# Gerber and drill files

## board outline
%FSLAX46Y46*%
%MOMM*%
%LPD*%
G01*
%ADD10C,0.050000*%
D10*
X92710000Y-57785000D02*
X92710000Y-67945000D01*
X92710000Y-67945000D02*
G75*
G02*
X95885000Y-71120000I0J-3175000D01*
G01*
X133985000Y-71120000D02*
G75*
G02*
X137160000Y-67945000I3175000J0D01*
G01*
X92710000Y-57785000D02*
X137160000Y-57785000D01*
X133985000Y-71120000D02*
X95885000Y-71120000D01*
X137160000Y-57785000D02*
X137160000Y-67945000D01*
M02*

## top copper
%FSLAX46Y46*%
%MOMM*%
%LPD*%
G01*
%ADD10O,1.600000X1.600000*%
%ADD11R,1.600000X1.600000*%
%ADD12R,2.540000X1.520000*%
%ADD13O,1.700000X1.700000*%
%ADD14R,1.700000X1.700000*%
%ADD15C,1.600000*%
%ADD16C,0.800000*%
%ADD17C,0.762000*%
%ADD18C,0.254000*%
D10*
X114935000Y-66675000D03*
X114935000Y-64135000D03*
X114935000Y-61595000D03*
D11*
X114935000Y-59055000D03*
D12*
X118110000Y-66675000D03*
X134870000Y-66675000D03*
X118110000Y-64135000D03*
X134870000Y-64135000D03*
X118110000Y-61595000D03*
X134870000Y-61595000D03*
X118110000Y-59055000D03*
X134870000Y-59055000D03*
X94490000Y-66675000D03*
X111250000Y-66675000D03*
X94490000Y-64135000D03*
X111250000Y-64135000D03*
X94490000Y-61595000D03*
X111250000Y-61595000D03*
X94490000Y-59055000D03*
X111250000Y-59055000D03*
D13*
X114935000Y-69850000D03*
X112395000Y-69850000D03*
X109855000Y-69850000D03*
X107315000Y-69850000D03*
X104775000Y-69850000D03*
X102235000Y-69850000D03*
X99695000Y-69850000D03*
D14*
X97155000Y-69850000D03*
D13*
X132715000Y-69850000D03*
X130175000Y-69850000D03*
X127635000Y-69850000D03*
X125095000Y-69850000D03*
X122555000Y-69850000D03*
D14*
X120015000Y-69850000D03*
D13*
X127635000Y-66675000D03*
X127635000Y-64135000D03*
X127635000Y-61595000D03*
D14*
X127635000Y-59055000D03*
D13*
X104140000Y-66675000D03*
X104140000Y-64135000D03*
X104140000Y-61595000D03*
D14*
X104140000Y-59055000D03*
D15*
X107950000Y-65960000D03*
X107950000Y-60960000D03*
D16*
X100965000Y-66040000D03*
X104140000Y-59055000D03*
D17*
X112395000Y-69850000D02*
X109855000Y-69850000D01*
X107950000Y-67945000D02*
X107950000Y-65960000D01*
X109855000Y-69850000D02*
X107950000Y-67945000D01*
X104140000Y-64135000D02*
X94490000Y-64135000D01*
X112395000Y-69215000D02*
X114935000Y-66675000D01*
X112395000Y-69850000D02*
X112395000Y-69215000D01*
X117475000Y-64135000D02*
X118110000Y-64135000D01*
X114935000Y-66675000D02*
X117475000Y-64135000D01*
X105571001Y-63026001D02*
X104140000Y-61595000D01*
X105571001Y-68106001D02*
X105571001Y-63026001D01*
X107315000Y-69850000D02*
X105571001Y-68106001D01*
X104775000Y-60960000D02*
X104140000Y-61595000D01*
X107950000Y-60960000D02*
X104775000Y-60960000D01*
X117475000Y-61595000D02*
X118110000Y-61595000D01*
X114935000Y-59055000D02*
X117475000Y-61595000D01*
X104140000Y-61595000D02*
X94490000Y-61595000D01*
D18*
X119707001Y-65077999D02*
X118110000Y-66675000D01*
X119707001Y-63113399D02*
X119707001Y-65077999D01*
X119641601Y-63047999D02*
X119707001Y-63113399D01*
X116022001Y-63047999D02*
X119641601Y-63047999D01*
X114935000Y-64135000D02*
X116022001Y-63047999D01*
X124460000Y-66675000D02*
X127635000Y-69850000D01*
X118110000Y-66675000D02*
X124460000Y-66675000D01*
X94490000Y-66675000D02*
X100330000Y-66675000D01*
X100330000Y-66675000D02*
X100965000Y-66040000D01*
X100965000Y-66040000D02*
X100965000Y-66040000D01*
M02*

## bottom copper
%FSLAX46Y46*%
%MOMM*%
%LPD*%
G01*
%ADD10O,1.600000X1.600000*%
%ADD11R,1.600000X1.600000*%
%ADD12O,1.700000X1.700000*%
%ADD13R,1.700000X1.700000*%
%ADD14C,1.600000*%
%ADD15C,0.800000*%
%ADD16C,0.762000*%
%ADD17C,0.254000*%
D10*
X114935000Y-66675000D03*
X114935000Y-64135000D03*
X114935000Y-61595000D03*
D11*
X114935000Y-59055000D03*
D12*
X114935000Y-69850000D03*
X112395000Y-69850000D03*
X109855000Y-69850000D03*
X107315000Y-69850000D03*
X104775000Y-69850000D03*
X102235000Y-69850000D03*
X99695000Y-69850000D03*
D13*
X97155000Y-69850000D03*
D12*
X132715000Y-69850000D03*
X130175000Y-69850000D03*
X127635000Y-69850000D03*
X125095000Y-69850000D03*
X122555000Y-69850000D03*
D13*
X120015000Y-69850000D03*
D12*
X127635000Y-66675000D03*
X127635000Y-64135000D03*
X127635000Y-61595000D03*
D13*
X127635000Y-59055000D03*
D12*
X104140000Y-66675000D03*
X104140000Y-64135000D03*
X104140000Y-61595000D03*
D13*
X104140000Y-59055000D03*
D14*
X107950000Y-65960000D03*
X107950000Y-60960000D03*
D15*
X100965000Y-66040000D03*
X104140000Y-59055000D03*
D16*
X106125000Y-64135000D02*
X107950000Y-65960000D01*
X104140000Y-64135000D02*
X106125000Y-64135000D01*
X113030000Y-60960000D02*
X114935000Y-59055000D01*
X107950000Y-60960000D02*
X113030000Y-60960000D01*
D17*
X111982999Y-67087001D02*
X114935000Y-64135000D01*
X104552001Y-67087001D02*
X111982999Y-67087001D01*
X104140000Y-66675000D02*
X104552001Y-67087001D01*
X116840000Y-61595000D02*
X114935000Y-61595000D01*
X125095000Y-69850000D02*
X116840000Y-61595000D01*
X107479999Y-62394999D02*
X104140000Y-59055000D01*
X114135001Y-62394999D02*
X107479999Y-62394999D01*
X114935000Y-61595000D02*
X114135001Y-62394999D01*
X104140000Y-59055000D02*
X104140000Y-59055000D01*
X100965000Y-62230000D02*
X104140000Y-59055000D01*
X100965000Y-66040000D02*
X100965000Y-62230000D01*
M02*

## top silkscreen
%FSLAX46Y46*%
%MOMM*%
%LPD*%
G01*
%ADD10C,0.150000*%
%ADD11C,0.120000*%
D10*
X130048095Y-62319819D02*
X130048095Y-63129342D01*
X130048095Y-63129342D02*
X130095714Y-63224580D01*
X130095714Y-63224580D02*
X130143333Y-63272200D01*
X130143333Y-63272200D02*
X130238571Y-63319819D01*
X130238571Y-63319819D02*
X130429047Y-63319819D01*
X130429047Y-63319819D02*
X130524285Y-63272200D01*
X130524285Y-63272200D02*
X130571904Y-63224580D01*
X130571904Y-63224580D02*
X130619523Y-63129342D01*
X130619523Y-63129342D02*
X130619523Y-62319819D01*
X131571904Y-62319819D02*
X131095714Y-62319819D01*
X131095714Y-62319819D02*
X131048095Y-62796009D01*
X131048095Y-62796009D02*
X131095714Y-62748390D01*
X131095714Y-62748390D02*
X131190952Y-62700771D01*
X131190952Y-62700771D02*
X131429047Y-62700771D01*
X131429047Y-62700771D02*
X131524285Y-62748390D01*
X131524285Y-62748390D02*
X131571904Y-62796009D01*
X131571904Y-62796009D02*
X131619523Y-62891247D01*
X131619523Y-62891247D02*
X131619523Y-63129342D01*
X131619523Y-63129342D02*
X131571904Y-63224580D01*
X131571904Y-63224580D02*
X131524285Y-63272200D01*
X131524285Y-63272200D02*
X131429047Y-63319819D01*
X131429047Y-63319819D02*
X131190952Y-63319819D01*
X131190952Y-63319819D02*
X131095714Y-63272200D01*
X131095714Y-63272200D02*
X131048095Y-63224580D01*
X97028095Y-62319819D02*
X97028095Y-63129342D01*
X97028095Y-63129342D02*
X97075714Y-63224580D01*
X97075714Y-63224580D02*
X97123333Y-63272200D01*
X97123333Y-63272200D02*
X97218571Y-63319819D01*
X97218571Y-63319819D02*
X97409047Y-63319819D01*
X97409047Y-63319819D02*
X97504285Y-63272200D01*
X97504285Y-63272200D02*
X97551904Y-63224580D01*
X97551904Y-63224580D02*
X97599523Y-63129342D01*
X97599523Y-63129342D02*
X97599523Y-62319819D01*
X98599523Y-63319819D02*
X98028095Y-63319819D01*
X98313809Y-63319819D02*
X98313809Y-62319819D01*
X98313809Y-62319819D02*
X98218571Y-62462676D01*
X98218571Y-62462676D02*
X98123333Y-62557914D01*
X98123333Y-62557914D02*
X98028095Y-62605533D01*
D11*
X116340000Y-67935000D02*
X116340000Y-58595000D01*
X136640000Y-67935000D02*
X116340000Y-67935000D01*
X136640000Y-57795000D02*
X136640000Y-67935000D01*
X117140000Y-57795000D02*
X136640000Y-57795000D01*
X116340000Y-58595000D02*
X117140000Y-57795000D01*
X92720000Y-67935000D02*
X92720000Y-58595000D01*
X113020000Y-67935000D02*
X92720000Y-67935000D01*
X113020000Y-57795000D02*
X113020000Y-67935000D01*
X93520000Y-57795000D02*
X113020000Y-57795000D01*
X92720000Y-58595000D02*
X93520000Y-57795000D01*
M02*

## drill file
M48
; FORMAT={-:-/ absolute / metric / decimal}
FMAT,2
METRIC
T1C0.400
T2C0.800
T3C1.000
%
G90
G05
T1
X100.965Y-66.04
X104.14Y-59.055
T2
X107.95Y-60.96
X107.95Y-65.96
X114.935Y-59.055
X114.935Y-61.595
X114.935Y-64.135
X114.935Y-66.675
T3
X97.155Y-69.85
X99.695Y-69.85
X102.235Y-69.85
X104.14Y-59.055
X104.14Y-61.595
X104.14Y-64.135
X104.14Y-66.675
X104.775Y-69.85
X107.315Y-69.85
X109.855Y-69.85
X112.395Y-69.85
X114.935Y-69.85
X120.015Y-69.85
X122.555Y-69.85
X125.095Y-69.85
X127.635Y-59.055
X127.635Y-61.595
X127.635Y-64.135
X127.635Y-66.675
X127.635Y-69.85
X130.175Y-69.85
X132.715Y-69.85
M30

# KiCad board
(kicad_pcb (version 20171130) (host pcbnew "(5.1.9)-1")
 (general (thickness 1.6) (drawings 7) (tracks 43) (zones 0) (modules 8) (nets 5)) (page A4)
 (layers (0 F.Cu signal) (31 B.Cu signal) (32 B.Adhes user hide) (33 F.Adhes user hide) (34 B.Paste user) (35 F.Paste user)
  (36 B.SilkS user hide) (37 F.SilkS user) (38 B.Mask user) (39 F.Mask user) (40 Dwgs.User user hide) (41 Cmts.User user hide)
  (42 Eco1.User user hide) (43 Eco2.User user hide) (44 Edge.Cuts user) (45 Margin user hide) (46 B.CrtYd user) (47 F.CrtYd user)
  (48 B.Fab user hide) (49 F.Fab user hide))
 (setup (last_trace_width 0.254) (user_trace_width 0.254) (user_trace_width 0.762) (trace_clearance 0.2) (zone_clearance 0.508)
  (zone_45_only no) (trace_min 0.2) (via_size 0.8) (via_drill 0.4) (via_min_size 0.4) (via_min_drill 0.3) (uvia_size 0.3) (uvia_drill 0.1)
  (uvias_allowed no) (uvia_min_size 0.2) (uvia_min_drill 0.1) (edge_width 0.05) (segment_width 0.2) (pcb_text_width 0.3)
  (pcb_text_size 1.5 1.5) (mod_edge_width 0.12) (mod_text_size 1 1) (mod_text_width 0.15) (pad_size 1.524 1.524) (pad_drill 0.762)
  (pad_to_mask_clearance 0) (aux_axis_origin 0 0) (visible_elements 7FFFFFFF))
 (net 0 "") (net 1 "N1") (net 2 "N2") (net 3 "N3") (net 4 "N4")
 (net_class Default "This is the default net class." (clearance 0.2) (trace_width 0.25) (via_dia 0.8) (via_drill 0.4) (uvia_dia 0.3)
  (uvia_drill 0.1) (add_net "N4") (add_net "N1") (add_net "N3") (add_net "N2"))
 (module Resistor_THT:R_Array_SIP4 (layer B.Cu) (at 114.935 59.055 270)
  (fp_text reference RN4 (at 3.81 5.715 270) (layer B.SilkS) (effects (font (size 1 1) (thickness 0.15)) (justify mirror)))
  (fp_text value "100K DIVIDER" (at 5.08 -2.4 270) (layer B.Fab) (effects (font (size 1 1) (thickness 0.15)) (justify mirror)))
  (pad 4 thru_hole oval (at 7.62 0 270) (size 1.6 1.6) (drill 0.8) (layers *.Cu *.Mask) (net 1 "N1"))
  (pad 3 thru_hole oval (at 5.08 0 270) (size 1.6 1.6) (drill 0.8) (layers *.Cu *.Mask) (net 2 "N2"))
  (pad 2 thru_hole oval (at 2.54 0 270) (size 1.6 1.6) (drill 0.8) (layers *.Cu *.Mask) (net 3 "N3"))
  (pad 1 thru_hole rect (at 0 0 270) (size 1.6 1.6) (drill 0.8) (layers *.Cu *.Mask) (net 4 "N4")))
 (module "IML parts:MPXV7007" (layer F.Cu) (at 126.49 62.865 270)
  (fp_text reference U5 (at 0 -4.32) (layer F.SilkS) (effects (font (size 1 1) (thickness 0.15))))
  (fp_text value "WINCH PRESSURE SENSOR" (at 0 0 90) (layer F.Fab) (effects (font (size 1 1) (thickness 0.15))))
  (fp_line (start 5.07 10.15) (end -4.27 10.15) (layer F.SilkS) (width 0.12))
  (fp_line (start 5.07 -10.15) (end 5.07 10.15) (layer F.SilkS) (width 0.12))
  (fp_line (start -5.07 -10.15) (end 5.07 -10.15) (layer F.SilkS) (width 0.12))
  (fp_line (start -5.07 9.35) (end -5.07 -10.15) (layer F.SilkS) (width 0.12))
  (fp_line (start -4.27 10.15) (end -5.07 9.35) (layer F.SilkS) (width 0.12))
  (pad 4 smd rect (at 3.81 8.38 270) (size 1.52 2.54) (layers F.Cu F.Paste F.Mask) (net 2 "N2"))
  (pad 5 smd rect (at 3.81 -8.38 270) (size 1.52 2.54) (layers F.Cu F.Paste F.Mask))
  (pad 3 smd rect (at 1.27 8.38 270) (size 1.52 2.54) (layers F.Cu F.Paste F.Mask) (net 1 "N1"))
  (pad 6 smd rect (at 1.27 -8.38 270) (size 1.52 2.54) (layers F.Cu F.Paste F.Mask))
  (pad 2 smd rect (at -1.27 8.38 270) (size 1.52 2.54) (layers F.Cu F.Paste F.Mask) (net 4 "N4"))
  (pad 7 smd rect (at -1.27 -8.38 270) (size 1.52 2.54) (layers F.Cu F.Paste F.Mask))
  (pad 1 smd rect (at -3.81 8.38 270) (size 1.52 2.54) (layers F.Cu F.Paste F.Mask))
  (pad 8 smd rect (at -3.81 -8.38 270) (size 1.52 2.54) (layers F.Cu F.Paste F.Mask)))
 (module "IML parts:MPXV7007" (layer F.Cu) (at 102.87 62.865 270)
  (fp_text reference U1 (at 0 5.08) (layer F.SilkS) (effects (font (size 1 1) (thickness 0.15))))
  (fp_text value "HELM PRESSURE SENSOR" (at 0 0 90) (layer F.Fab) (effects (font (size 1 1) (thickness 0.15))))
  (fp_line (start 5.07 10.15) (end -4.27 10.15) (layer F.SilkS) (width 0.12))
  (fp_line (start 5.07 -10.15) (end 5.07 10.15) (layer F.SilkS) (width 0.12))
  (fp_line (start -5.07 -10.15) (end 5.07 -10.15) (layer F.SilkS) (width 0.12))
  (fp_line (start -5.07 9.35) (end -5.07 -10.15) (layer F.SilkS) (width 0.12))
  (fp_line (start -4.27 10.15) (end -5.07 9.35) (layer F.SilkS) (width 0.12))
  (pad 4 smd rect (at 3.81 8.38 270) (size 1.52 2.54) (layers F.Cu F.Paste F.Mask) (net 3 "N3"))
  (pad 5 smd rect (at 3.81 -8.38 270) (size 1.52 2.54) (layers F.Cu F.Paste F.Mask))
  (pad 3 smd rect (at 1.27 8.38 270) (size 1.52 2.54) (layers F.Cu F.Paste F.Mask) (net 1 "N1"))
  (pad 6 smd rect (at 1.27 -8.38 270) (size 1.52 2.54) (layers F.Cu F.Paste F.Mask))
  (pad 2 smd rect (at -1.27 8.38 270) (size 1.52 2.54) (layers F.Cu F.Paste F.Mask) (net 4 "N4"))
  (pad 7 smd rect (at -1.27 -8.38 270) (size 1.52 2.54) (layers F.Cu F.Paste F.Mask))
  (pad 1 smd rect (at -3.81 8.38 270) (size 1.52 2.54) (layers F.Cu F.Paste F.Mask))
  (pad 8 smd rect (at -3.81 -8.38 270) (size 1.52 2.54) (layers F.Cu F.Paste F.Mask)))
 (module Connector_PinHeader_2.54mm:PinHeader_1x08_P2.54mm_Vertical (layer B.Cu) (at 97.155 69.85 270)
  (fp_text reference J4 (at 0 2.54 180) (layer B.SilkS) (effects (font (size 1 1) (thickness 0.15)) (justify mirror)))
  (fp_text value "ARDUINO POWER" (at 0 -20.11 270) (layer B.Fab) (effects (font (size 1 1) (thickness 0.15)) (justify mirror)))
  (pad 8 thru_hole oval (at 0 -17.78 270) (size 1.7 1.7) (drill 1) (layers *.Cu *.Mask))
  (pad 7 thru_hole oval (at 0 -15.24 270) (size 1.7 1.7) (drill 1) (layers *.Cu *.Mask) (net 1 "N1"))
  (pad 6 thru_hole oval (at 0 -12.7 270) (size 1.7 1.7) (drill 1) (layers *.Cu *.Mask) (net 1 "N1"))
  (pad 5 thru_hole oval (at 0 -10.16 270) (size 1.7 1.7) (drill 1) (layers *.Cu *.Mask) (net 4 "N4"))
  (pad 4 thru_hole oval (at 0 -7.62 270) (size 1.7 1.7) (drill 1) (layers *.Cu *.Mask))
  (pad 3 thru_hole oval (at 0 -5.08 270) (size 1.7 1.7) (drill 1) (layers *.Cu *.Mask))
  (pad 2 thru_hole oval (at 0 -2.54 270) (size 1.7 1.7) (drill 1) (layers *.Cu *.Mask))
  (pad 1 thru_hole rect (at 0 0 270) (size 1.7 1.7) (drill 1) (layers *.Cu *.Mask)))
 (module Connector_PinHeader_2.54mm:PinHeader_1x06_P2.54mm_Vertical (layer B.Cu) (at 120.015 69.85 270)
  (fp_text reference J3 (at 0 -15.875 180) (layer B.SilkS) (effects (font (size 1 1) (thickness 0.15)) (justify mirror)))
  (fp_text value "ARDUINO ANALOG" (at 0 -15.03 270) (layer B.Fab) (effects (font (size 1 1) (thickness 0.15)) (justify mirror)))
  (pad 6 thru_hole oval (at 0 -12.7 270) (size 1.7 1.7) (drill 1) (layers *.Cu *.Mask))
  (pad 5 thru_hole oval (at 0 -10.16 270) (size 1.7 1.7) (drill 1) (layers *.Cu *.Mask))
  (pad 4 thru_hole oval (at 0 -7.62 270) (size 1.7 1.7) (drill 1) (layers *.Cu *.Mask) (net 2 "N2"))
  (pad 3 thru_hole oval (at 0 -5.08 270) (size 1.7 1.7) (drill 1) (layers *.Cu *.Mask) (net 3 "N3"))
  (pad 2 thru_hole oval (at 0 -2.54 270) (size 1.7 1.7) (drill 1) (layers *.Cu *.Mask))
  (pad 1 thru_hole rect (at 0 0 270) (size 1.7 1.7) (drill 1) (layers *.Cu *.Mask)))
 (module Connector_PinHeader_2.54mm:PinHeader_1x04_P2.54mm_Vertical (layer B.Cu) (at 127.635 59.055 180)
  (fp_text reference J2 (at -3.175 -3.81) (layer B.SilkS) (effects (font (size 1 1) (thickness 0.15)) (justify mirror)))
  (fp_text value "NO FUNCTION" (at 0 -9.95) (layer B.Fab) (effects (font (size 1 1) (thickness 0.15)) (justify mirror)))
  (pad 4 thru_hole oval (at 0 -7.62 180) (size 1.7 1.7) (drill 1) (layers *.Cu *.Mask))
  (pad 3 thru_hole oval (at 0 -5.08 180) (size 1.7 1.7) (drill 1) (layers *.Cu *.Mask))
  (pad 2 thru_hole oval (at 0 -2.54 180) (size 1.7 1.7) (drill 1) (layers *.Cu *.Mask))
  (pad 1 thru_hole rect (at 0 0 180) (size 1.7 1.7) (drill 1) (layers *.Cu *.Mask)))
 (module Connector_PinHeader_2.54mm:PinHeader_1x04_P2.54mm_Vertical (layer B.Cu) (at 104.14 59.055 180)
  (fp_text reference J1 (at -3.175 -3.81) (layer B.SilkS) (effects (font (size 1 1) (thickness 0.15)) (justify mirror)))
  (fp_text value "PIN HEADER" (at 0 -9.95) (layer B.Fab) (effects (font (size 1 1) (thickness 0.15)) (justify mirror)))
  (pad 4 thru_hole oval (at 0 -7.62 180) (size 1.7 1.7) (drill 1) (layers *.Cu *.Mask) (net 2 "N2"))
  (pad 3 thru_hole oval (at 0 -5.08 180) (size 1.7 1.7) (drill 1) (layers *.Cu *.Mask) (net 1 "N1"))
  (pad 2 thru_hole oval (at 0 -2.54 180) (size 1.7 1.7) (drill 1) (layers *.Cu *.Mask) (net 4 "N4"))
  (pad 1 thru_hole rect (at 0 0 180) (size 1.7 1.7) (drill 1) (layers *.Cu *.Mask) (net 3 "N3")))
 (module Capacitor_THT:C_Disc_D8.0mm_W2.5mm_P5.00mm (layer B.Cu) (at 107.95 60.96 270)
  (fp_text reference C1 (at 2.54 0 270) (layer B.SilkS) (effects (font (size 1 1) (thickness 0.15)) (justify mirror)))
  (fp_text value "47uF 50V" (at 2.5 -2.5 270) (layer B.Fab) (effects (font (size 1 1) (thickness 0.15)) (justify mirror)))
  (pad 2 thru_hole circle (at 5 0 270) (size 1.6 1.6) (drill 0.8) (layers *.Cu *.Mask) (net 1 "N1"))
  (pad 1 thru_hole circle (at 0 0 270) (size 1.6 1.6) (drill 0.8) (layers *.Cu *.Mask) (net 4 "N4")))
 (gr_line (start 92.71 57.785) (end 92.71 67.945) (layer Edge.Cuts) (width 0.05))
 (gr_arc (start 92.71 71.12) (end 95.885 71.12) (angle -90) (layer Edge.Cuts) (width 0.05))
 (gr_arc (start 137.16 71.12) (end 137.16 67.945) (angle -90) (layer Edge.Cuts) (width 0.05))
 (gr_line (start 92.71 57.785) (end 137.16 57.785) (layer Edge.Cuts) (width 0.05))
 (gr_line (start 133.985 71.12) (end 95.885 71.12) (layer Edge.Cuts) (width 0.05))
 (gr_line (start 137.16 57.785) (end 137.16 67.945) (layer Edge.Cuts) (width 0.05))
 (segment (start 112.395 69.85) (end 109.855 69.85) (width 0.762) (layer F.Cu) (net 1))
 (segment (start 107.95 67.945) (end 107.95 65.96) (width 0.762) (layer F.Cu) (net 1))
 (segment (start 109.855 69.85) (end 107.95 67.945) (width 0.762) (layer F.Cu) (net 1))
 (segment (start 104.14 64.135) (end 94.49 64.135) (width 0.762) (layer F.Cu) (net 1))
 (segment (start 112.395 69.215) (end 114.935 66.675) (width 0.762) (layer F.Cu) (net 1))
 (segment (start 112.395 69.85) (end 112.395 69.215) (width 0.762) (layer F.Cu) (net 1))
 (segment (start 117.475 64.135) (end 118.11 64.135) (width 0.762) (layer F.Cu) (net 1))
 (segment (start 114.935 66.675) (end 117.475 64.135) (width 0.762) (layer F.Cu) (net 1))
 (segment (start 106.125 64.135) (end 107.95 65.96) (width 0.762) (layer B.Cu) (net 1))
 (segment (start 104.14 64.135) (end 106.125 64.135) (width 0.762) (layer B.Cu) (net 1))
 (segment (start 105.571001 63.026001) (end 104.14 61.595) (width 0.762) (layer F.Cu) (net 4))
 (segment (start 105.571001 68.106001) (end 105.571001 63.026001) (width 0.762) (layer F.Cu) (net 4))
 (segment (start 107.315 69.85) (end 105.571001 68.106001) (width 0.762) (layer F.Cu) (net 4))
 (segment (start 104.775 60.96) (end 104.14 61.595) (width 0.762) (layer F.Cu) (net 4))
 (segment (start 107.95 60.96) (end 104.775 60.96) (width 0.762) (layer F.Cu) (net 4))
 (segment (start 113.03 60.96) (end 114.935 59.055) (width 0.762) (layer B.Cu) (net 4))
 (segment (start 107.95 60.96) (end 113.03 60.96) (width 0.762) (layer B.Cu) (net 4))
 (segment (start 117.475 61.595) (end 118.11 61.595) (width 0.762) (layer F.Cu) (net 4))
 (segment (start 114.935 59.055) (end 117.475 61.595) (width 0.762) (layer F.Cu) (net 4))
 (segment (start 104.14 61.595) (end 94.49 61.595) (width 0.762) (layer F.Cu) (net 4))
 (segment (start 111.982999 67.087001) (end 114.935 64.135) (width 0.254) (layer B.Cu) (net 2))
 (segment (start 104.552001 67.087001) (end 111.982999 67.087001) (width 0.254) (layer B.Cu) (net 2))
 (segment (start 104.14 66.675) (end 104.552001 67.087001) (width 0.254) (layer B.Cu) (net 2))
 (segment (start 119.707001 65.077999) (end 118.11 66.675) (width 0.254) (layer F.Cu) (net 2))
 (segment (start 119.707001 63.113399) (end 119.707001 65.077999) (width 0.254) (layer F.Cu) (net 2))
 (segment (start 119.641601 63.047999) (end 119.707001 63.113399) (width 0.254) (layer F.Cu) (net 2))
 (segment (start 116.022001 63.047999) (end 119.641601 63.047999) (width 0.254) (layer F.Cu) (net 2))
 (segment (start 114.935 64.135) (end 116.022001 63.047999) (width 0.254) (layer F.Cu) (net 2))
 (segment (start 124.46 66.675) (end 127.635 69.85) (width 0.254) (layer F.Cu) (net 2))
 (segment (start 118.11 66.675) (end 124.46 66.675) (width 0.254) (layer F.Cu) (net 2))
 (segment (start 116.84 61.595) (end 114.935 61.595) (width 0.254) (layer B.Cu) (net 3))
 (segment (start 125.095 69.85) (end 116.84 61.595) (width 0.254) (layer B.Cu) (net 3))
 (segment (start 107.479999 62.394999) (end 104.14 59.055) (width 0.254) (layer B.Cu) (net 3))
 (segment (start 114.135001 62.394999) (end 107.479999 62.394999) (width 0.254) (layer B.Cu) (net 3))
 (segment (start 114.935 61.595) (end 114.135001 62.394999) (width 0.254) (layer B.Cu) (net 3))
 (segment (start 94.49 66.675) (end 100.33 66.675) (width 0.254) (layer F.Cu) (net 3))
 (segment (start 100.33 66.675) (end 100.965 66.04) (width 0.254) (layer F.Cu) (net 3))
 (segment (start 100.965 66.04) (end 100.965 66.04) (width 0.254) (layer F.Cu) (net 3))
 (via (at 100.965 66.04) (size 0.8) (drill 0.4) (layers F.Cu B.Cu) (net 3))
 (segment (start 104.14 59.055) (end 104.14 59.055) (width 0.254) (layer B.Cu) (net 3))
 (via (at 104.14 59.055) (size 0.8) (drill 0.4) (layers F.Cu B.Cu) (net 3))
 (segment (start 100.965 62.23) (end 104.14 59.055) (width 0.254) (layer B.Cu) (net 3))
 (segment (start 100.965 66.04) (end 100.965 62.23) (width 0.254) (layer B.Cu) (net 3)))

